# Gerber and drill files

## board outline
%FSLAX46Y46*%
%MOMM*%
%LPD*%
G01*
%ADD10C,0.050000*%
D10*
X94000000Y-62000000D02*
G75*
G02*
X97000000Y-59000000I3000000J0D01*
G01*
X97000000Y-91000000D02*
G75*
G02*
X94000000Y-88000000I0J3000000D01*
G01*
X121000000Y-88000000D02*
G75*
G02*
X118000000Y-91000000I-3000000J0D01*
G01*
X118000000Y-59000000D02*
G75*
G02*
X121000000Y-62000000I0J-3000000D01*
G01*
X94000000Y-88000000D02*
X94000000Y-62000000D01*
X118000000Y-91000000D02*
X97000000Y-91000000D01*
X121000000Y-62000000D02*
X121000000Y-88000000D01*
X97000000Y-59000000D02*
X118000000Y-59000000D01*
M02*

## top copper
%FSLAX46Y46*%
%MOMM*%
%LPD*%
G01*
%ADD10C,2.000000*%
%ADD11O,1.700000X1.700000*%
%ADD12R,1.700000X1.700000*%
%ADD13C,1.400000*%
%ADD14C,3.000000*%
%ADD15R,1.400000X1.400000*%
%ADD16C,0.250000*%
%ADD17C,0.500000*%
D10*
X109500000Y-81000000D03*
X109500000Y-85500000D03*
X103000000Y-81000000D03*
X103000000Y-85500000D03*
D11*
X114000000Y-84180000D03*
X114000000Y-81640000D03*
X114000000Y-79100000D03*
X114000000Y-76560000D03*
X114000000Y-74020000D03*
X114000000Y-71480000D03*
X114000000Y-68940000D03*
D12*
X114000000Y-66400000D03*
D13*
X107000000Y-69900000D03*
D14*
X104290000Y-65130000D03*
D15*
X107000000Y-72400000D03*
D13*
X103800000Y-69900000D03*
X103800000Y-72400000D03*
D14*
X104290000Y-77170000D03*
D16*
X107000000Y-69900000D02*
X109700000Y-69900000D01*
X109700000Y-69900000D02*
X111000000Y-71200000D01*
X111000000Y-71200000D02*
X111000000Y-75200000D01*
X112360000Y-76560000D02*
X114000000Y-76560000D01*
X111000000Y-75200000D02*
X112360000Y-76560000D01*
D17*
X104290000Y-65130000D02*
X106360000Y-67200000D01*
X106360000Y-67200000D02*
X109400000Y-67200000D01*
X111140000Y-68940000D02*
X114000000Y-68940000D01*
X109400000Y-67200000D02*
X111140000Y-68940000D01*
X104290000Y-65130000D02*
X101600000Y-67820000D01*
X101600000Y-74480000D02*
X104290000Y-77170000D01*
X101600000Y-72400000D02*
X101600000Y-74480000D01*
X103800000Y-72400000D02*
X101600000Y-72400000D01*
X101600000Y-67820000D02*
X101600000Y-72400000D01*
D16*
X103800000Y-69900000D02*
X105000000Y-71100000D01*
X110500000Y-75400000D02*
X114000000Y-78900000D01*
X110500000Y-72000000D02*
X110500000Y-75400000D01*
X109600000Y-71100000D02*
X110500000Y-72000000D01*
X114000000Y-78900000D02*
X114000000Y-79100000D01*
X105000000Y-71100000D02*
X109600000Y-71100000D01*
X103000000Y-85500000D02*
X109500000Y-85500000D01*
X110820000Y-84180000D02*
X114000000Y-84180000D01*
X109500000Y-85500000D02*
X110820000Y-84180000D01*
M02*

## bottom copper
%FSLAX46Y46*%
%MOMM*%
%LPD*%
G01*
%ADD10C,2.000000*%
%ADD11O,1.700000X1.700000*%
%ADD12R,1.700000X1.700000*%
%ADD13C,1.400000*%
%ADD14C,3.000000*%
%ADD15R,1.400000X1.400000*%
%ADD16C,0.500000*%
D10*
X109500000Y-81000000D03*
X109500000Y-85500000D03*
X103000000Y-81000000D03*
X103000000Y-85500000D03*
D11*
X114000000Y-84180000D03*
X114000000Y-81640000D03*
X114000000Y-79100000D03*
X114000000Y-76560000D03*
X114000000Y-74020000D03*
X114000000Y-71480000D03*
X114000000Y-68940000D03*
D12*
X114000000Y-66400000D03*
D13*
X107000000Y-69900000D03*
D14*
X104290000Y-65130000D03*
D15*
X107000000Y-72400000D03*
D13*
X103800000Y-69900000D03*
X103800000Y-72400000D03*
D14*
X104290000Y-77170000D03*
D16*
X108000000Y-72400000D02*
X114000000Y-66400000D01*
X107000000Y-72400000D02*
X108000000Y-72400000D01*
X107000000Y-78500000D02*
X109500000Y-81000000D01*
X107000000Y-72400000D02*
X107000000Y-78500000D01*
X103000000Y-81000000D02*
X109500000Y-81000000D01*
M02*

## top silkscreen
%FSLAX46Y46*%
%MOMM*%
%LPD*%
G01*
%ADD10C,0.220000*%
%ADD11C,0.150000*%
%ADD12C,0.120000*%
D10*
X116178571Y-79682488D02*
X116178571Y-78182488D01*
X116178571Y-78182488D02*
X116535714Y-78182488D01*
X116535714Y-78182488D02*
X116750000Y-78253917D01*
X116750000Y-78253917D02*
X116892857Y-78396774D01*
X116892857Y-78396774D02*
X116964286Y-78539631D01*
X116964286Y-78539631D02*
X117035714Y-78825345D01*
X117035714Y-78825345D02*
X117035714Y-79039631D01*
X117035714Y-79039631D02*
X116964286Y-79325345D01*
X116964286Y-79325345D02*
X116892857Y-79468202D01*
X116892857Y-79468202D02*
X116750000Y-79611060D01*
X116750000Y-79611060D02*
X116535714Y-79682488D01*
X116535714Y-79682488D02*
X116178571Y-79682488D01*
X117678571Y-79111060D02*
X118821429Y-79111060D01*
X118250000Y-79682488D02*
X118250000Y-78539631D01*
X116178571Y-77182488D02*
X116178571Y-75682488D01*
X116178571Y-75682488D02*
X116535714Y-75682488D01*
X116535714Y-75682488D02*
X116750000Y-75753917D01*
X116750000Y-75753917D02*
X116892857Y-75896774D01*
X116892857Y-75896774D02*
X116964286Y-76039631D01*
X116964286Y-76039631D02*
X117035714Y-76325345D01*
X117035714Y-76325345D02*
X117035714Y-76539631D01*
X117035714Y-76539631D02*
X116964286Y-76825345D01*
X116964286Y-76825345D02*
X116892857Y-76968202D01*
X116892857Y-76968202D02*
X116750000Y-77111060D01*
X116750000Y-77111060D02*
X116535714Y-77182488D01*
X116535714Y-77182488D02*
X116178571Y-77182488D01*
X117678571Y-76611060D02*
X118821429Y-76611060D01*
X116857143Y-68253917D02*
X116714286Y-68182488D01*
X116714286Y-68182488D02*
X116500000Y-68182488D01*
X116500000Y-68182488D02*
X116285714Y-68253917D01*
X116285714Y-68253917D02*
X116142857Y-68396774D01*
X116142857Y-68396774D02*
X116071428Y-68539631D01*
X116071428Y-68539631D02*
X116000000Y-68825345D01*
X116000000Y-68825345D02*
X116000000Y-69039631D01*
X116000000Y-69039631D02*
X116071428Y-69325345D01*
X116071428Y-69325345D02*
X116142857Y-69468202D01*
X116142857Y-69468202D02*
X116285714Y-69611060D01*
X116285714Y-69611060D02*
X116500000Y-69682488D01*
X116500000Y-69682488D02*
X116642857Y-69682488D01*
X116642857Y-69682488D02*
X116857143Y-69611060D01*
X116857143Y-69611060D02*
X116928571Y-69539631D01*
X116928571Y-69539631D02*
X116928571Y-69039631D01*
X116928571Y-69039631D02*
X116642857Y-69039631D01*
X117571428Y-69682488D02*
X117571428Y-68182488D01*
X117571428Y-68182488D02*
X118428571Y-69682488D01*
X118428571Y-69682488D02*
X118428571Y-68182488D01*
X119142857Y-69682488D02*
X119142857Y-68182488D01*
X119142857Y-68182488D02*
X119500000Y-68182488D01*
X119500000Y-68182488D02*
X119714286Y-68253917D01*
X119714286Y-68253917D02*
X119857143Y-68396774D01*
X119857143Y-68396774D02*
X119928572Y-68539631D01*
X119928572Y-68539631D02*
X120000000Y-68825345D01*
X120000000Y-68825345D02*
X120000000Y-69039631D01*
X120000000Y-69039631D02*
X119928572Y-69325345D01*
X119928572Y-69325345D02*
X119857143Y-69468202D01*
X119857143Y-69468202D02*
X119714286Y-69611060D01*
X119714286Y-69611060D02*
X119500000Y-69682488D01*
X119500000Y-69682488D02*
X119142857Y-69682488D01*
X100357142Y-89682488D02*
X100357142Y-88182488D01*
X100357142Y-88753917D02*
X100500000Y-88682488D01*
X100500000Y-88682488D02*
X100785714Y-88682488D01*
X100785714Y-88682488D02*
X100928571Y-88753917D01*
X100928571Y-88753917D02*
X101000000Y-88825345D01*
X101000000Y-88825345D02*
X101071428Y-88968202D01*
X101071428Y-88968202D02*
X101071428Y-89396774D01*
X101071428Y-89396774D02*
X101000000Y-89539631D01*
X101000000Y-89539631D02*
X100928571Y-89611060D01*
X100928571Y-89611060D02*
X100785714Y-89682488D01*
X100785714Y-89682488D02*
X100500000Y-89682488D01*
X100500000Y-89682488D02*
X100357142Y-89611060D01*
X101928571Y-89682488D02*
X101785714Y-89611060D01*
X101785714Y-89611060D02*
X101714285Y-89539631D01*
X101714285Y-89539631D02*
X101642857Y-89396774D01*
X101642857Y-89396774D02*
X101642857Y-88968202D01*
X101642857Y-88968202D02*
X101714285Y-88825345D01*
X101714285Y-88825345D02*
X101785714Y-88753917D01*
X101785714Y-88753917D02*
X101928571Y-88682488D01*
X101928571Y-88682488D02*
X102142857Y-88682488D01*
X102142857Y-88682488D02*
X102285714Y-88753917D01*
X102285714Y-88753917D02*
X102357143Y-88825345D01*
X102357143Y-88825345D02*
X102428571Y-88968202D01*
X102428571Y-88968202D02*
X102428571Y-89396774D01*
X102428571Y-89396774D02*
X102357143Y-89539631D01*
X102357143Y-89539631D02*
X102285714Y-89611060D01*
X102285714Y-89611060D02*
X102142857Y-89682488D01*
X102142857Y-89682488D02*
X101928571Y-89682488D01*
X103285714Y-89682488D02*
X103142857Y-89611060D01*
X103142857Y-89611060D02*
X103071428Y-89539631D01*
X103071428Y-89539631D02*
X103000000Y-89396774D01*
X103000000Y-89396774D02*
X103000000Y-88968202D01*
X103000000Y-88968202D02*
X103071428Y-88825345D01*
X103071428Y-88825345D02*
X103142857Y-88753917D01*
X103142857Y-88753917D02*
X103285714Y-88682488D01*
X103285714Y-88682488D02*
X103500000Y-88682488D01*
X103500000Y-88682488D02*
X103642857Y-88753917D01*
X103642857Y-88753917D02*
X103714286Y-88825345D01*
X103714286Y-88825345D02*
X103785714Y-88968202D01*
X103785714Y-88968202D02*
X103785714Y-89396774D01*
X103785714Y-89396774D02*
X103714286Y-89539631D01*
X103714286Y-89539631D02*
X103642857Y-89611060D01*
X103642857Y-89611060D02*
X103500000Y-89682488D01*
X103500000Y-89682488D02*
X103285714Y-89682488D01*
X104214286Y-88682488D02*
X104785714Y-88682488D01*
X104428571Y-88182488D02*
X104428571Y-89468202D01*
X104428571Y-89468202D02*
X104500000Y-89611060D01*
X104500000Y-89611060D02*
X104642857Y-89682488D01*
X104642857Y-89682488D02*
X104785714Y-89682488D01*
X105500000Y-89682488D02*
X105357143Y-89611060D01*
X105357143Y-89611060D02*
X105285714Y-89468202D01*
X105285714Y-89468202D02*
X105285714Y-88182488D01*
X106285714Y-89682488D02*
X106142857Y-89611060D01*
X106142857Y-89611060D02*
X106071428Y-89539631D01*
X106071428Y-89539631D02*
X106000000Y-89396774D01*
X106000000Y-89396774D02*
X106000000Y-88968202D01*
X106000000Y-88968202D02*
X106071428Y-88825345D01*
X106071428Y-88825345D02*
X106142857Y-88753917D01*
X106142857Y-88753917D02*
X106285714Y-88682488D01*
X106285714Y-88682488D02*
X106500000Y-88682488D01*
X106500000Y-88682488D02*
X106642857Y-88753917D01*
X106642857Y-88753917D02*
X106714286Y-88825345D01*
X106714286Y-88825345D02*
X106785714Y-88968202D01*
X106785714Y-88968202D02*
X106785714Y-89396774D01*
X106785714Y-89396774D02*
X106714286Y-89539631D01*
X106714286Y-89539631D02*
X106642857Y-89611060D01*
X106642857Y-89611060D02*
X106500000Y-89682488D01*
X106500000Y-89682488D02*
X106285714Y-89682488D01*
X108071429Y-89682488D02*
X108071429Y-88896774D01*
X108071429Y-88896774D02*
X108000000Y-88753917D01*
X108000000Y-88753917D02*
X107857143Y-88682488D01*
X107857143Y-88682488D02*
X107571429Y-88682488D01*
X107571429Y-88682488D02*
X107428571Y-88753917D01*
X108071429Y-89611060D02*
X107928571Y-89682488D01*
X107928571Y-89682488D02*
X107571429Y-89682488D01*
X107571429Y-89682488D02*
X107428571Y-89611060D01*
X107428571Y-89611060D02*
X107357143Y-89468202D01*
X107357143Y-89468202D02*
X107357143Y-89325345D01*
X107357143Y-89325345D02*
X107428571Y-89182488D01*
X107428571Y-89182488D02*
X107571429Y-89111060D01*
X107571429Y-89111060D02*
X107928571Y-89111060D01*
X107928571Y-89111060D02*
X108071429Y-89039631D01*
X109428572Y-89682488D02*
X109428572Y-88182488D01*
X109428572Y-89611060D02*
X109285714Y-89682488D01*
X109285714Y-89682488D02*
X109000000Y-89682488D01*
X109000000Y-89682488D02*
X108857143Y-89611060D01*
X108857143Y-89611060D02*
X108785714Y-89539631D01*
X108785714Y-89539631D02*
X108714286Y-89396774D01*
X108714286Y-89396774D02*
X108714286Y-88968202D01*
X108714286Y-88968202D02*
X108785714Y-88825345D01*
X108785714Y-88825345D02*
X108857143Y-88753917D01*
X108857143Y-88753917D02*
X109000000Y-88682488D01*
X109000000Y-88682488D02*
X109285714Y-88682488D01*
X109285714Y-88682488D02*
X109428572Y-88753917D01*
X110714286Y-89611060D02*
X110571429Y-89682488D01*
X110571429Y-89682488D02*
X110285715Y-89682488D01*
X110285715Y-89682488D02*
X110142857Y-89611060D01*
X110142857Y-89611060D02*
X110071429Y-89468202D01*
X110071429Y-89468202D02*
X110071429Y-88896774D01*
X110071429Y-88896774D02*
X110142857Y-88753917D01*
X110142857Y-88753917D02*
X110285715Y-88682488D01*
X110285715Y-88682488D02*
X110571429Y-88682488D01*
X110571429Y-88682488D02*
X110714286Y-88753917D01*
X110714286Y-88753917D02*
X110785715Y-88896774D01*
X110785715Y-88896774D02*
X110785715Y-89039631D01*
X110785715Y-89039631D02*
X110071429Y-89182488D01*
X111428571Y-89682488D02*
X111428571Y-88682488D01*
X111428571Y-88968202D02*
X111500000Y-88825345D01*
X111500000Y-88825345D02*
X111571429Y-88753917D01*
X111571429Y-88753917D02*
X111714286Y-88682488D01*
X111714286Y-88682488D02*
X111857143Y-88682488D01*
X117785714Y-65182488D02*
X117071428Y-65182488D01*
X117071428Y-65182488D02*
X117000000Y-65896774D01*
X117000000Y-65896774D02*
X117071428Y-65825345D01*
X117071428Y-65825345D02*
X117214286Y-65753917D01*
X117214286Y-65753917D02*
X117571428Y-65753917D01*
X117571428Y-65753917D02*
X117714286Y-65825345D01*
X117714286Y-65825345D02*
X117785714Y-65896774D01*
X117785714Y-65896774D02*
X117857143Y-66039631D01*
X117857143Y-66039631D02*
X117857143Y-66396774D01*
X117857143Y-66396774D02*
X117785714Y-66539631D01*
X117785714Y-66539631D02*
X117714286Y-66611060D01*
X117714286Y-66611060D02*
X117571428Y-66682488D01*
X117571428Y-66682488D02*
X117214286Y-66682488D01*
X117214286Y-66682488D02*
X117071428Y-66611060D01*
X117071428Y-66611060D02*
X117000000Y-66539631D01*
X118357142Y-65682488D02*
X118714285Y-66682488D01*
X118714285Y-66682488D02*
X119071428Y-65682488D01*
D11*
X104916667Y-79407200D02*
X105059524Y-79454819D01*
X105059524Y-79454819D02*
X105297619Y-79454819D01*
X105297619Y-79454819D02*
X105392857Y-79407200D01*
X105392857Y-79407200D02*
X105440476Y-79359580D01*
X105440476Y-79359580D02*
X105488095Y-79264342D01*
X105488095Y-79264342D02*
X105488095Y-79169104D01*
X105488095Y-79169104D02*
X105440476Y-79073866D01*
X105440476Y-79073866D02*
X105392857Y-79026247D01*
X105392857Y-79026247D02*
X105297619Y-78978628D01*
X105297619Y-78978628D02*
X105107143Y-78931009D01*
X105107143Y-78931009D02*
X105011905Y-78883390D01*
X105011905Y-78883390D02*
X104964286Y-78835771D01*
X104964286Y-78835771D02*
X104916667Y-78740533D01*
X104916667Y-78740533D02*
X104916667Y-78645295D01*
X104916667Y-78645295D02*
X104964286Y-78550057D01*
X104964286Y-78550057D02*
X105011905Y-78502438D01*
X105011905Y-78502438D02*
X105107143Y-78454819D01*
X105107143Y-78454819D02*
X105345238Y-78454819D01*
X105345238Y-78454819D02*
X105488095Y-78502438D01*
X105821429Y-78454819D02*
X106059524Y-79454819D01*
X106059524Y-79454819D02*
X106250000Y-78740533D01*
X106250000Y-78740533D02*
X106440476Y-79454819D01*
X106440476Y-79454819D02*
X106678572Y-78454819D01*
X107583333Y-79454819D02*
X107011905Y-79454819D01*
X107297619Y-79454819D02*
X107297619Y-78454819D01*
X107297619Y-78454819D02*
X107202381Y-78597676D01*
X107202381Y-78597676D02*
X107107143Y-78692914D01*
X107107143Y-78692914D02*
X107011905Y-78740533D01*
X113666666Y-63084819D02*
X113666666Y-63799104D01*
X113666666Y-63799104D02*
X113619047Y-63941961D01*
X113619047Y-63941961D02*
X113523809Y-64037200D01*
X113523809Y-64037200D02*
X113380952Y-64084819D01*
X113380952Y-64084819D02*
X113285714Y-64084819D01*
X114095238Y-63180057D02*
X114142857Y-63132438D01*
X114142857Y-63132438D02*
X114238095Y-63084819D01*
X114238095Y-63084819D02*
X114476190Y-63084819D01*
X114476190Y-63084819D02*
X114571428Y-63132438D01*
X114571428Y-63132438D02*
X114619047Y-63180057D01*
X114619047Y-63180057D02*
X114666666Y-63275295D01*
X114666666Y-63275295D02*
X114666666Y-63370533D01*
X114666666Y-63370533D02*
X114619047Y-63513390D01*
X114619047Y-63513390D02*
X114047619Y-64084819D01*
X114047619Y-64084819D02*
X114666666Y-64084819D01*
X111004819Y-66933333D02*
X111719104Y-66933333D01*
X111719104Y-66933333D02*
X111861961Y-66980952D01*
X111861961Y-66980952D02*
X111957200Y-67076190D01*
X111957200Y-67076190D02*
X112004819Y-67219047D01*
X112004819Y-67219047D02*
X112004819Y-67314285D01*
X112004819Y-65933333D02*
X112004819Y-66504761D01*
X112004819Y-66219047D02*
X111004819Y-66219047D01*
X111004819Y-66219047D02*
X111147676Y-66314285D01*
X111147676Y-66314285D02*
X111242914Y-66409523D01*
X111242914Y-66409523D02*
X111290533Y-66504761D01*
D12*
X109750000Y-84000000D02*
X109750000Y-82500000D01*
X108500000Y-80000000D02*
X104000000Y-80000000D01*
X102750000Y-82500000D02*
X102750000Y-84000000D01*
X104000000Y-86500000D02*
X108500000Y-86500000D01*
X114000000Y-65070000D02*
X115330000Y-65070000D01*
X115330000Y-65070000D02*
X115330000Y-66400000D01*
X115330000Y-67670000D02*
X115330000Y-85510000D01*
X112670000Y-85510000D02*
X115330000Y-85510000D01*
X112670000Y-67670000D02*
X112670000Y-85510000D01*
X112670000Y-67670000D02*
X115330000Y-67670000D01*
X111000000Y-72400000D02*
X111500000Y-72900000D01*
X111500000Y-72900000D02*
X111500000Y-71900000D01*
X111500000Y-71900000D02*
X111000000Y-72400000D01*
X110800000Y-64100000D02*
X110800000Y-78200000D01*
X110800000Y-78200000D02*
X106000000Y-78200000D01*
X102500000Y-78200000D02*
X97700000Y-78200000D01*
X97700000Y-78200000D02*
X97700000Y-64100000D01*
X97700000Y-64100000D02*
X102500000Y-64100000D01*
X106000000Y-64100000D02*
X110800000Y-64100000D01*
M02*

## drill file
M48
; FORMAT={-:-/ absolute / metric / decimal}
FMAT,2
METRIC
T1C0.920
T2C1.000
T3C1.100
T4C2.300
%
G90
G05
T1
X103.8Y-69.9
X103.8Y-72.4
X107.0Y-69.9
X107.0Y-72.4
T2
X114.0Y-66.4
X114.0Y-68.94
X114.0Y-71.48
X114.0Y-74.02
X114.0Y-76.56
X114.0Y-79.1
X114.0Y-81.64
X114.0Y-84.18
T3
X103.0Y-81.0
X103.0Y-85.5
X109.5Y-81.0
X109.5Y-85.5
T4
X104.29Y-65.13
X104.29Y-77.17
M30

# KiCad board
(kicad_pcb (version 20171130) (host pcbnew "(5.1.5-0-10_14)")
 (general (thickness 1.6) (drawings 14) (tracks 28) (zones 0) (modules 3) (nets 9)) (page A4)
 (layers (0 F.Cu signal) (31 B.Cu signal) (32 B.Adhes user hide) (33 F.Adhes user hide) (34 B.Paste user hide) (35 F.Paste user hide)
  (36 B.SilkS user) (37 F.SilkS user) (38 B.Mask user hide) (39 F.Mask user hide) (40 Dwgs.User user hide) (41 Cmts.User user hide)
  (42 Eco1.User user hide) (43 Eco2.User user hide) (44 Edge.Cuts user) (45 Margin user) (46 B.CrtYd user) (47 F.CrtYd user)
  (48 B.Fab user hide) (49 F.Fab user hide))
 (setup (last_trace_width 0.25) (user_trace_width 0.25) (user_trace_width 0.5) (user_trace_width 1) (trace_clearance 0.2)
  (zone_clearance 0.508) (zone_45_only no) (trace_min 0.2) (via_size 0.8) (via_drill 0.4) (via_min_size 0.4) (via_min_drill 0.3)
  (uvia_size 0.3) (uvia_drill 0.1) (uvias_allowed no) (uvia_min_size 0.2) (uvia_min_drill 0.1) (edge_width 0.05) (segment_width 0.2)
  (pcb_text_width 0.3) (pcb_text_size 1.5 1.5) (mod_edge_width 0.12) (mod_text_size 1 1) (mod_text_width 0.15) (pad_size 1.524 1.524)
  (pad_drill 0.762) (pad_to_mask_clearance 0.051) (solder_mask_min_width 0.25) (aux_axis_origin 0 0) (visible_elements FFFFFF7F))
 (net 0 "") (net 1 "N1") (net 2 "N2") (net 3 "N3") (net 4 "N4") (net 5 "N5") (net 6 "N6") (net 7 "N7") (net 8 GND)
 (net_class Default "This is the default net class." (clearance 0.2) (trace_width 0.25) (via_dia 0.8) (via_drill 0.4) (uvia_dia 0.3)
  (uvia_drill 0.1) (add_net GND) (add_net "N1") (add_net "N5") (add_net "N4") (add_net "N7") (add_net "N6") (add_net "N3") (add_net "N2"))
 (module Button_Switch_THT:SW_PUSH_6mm (layer F.Cu) (at 103 81)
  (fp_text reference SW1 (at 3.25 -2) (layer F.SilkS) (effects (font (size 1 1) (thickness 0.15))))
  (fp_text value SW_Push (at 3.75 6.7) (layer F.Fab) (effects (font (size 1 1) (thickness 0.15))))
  (fp_line (start 6.75 3) (end 6.75 1.5) (layer F.SilkS) (width 0.12))
  (fp_line (start 5.5 -1) (end 1 -1) (layer F.SilkS) (width 0.12))
  (fp_line (start -0.25 1.5) (end -0.25 3) (layer F.SilkS) (width 0.12))
  (fp_line (start 1 5.5) (end 5.5 5.5) (layer F.SilkS) (width 0.12))
  (pad 1 thru_hole circle (at 6.5 0 90) (size 2 2) (drill 1.1) (layers *.Cu *.Mask) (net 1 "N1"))
  (pad 2 thru_hole circle (at 6.5 4.5 90) (size 2 2) (drill 1.1) (layers *.Cu *.Mask) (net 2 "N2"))
  (pad 1 thru_hole circle (at 0 0 90) (size 2 2) (drill 1.1) (layers *.Cu *.Mask) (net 1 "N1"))
  (pad 2 thru_hole circle (at 0 4.5 90) (size 2 2) (drill 1.1) (layers *.Cu *.Mask) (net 2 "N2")))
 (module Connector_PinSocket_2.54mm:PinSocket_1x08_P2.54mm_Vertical (layer F.Cu) (at 114 66.4)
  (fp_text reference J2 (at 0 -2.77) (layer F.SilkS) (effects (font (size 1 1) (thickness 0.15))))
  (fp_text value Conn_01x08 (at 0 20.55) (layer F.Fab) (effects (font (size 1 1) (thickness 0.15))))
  (fp_line (start 0 -1.33) (end 1.33 -1.33) (layer F.SilkS) (width 0.12))
  (fp_line (start 1.33 -1.33) (end 1.33 0) (layer F.SilkS) (width 0.12))
  (fp_line (start 1.33 1.27) (end 1.33 19.11) (layer F.SilkS) (width 0.12))
  (fp_line (start -1.33 19.11) (end 1.33 19.11) (layer F.SilkS) (width 0.12))
  (fp_line (start -1.33 1.27) (end -1.33 19.11) (layer F.SilkS) (width 0.12))
  (fp_line (start -1.33 1.27) (end 1.33 1.27) (layer F.SilkS) (width 0.12))
  (pad 8 thru_hole oval (at 0 17.78) (size 1.7 1.7) (drill 1) (layers *.Cu *.Mask) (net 2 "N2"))
  (pad 7 thru_hole oval (at 0 15.24) (size 1.7 1.7) (drill 1) (layers *.Cu *.Mask) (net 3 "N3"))
  (pad 6 thru_hole oval (at 0 12.7) (size 1.7 1.7) (drill 1) (layers *.Cu *.Mask) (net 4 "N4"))
  (pad 5 thru_hole oval (at 0 10.16) (size 1.7 1.7) (drill 1) (layers *.Cu *.Mask) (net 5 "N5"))
  (pad 4 thru_hole oval (at 0 7.62) (size 1.7 1.7) (drill 1) (layers *.Cu *.Mask) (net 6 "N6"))
  (pad 3 thru_hole oval (at 0 5.08) (size 1.7 1.7) (drill 1) (layers *.Cu *.Mask) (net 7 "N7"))
  (pad 2 thru_hole oval (at 0 2.54) (size 1.7 1.7) (drill 1) (layers *.Cu *.Mask) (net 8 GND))
  (pad 1 thru_hole rect (at 0 0) (size 1.7 1.7) (drill 1) (layers *.Cu *.Mask) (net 1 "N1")))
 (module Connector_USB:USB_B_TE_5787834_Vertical (layer F.Cu) (at 107 72.4 270)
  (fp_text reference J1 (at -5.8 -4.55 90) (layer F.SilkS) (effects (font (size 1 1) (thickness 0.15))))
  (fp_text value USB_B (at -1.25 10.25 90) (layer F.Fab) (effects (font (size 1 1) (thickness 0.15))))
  (fp_line (start 0 -4) (end 0.5 -4.5) (layer F.SilkS) (width 0.12))
  (fp_line (start 0.5 -4.5) (end -0.5 -4.5) (layer F.SilkS) (width 0.12))
  (fp_line (start -0.5 -4.5) (end 0 -4) (layer F.SilkS) (width 0.12))
  (fp_line (start -8.3 -3.8) (end 5.8 -3.8) (layer F.SilkS) (width 0.12))
  (fp_line (start 5.8 -3.8) (end 5.8 1) (layer F.SilkS) (width 0.12))
  (fp_line (start 5.8 4.5) (end 5.8 9.3) (layer F.SilkS) (width 0.12))
  (fp_line (start 5.8 9.3) (end -8.3 9.3) (layer F.SilkS) (width 0.12))
  (fp_line (start -8.3 9.3) (end -8.3 4.5) (layer F.SilkS) (width 0.12))
  (fp_line (start -8.3 1) (end -8.3 -3.8) (layer F.SilkS) (width 0.12))
  (pad 2 thru_hole circle (at -2.5 0 270) (size 1.4 1.4) (drill 0.92) (layers *.Cu *.Mask) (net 5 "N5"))
  (pad 5 thru_hole circle (at -7.27 2.71 270) (size 3 3) (drill 2.3) (layers *.Cu *.Mask) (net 8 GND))
  (pad 1 thru_hole rect (at 0 0 270) (size 1.4 1.4) (drill 0.92) (layers *.Cu *.Mask) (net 1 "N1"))
  (pad 3 thru_hole circle (at -2.5 3.2 270) (size 1.4 1.4) (drill 0.92) (layers *.Cu *.Mask) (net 4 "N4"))
  (pad 4 thru_hole circle (at 0 3.2 270) (size 1.4 1.4) (drill 0.92) (layers *.Cu *.Mask) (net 8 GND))
  (pad 5 thru_hole circle (at 4.77 2.71 270) (size 3 3) (drill 2.3) (layers *.Cu *.Mask) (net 8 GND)))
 (gr_arc (start 97 62) (end 97 59) (angle -90) (layer Edge.Cuts) (width 0.05))
 (gr_arc (start 97 88) (end 94 88) (angle -90) (layer Edge.Cuts) (width 0.05))
 (gr_arc (start 118 88) (end 118 91) (angle -90) (layer Edge.Cuts) (width 0.05))
 (gr_arc (start 118 62) (end 121 62) (angle -90) (layer Edge.Cuts) (width 0.05))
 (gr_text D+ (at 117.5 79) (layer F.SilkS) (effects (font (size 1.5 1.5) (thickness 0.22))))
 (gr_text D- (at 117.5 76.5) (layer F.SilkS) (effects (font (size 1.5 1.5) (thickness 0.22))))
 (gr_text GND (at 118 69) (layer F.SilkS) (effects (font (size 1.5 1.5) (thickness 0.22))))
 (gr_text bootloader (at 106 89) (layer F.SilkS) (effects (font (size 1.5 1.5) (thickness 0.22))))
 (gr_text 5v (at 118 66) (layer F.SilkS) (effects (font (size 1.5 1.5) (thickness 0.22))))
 (gr_line (start 94 88) (end 94 62) (layer Edge.Cuts) (width 0.05))
 (gr_line (start 118 91) (end 97 91) (layer Edge.Cuts) (width 0.05))
 (gr_line (start 121 62) (end 121 88) (layer Edge.Cuts) (width 0.05))
 (gr_line (start 97 59) (end 118 59) (layer Edge.Cuts) (width 0.05))
 (segment (start 107 69.9) (end 109.7 69.9) (width 0.25) (layer F.Cu) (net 5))
 (segment (start 109.7 69.9) (end 111 71.2) (width 0.25) (layer F.Cu) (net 5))
 (segment (start 111 71.2) (end 111 75.2) (width 0.25) (layer F.Cu) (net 5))
 (segment (start 112.36 76.56) (end 114 76.56) (width 0.25) (layer F.Cu) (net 5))
 (segment (start 111 75.2) (end 112.36 76.56) (width 0.25) (layer F.Cu) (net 5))
 (segment (start 104.29 65.13) (end 106.36 67.2) (width 0.5) (layer F.Cu) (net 8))
 (segment (start 106.36 67.2) (end 109.4 67.2) (width 0.5) (layer F.Cu) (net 8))
 (segment (start 111.14 68.94) (end 114 68.94) (width 0.5) (layer F.Cu) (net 8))
 (segment (start 109.4 67.2) (end 111.14 68.94) (width 0.5) (layer F.Cu) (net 8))
 (segment (start 104.29 65.13) (end 101.6 67.82) (width 0.5) (layer F.Cu) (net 8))
 (segment (start 101.6 74.48) (end 104.29 77.17) (width 0.5) (layer F.Cu) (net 8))
 (segment (start 101.6 72.4) (end 101.6 74.48) (width 0.5) (layer F.Cu) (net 8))
 (segment (start 103.8 72.4) (end 101.6 72.4) (width 0.5) (layer F.Cu) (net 8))
 (segment (start 101.6 67.82) (end 101.6 72.4) (width 0.5) (layer F.Cu) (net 8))
 (segment (start 108 72.4) (end 114 66.4) (width 0.5) (layer B.Cu) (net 1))
 (segment (start 107 72.4) (end 108 72.4) (width 0.5) (layer B.Cu) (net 1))
 (segment (start 107 78.5) (end 109.5 81) (width 0.5) (layer B.Cu) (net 1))
 (segment (start 107 72.4) (end 107 78.5) (width 0.5) (layer B.Cu) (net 1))
 (segment (start 103 81) (end 109.5 81) (width 0.5) (layer B.Cu) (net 1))
 (segment (start 103.8 69.9) (end 105 71.1) (width 0.25) (layer F.Cu) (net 4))
 (segment (start 110.5 75.4) (end 114 78.9) (width 0.25) (layer F.Cu) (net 4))
 (segment (start 110.5 72) (end 110.5 75.4) (width 0.25) (layer F.Cu) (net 4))
 (segment (start 109.6 71.1) (end 110.5 72) (width 0.25) (layer F.Cu) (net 4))
 (segment (start 114 78.9) (end 114 79.1) (width 0.25) (layer F.Cu) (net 4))
 (segment (start 105 71.1) (end 109.6 71.1) (width 0.25) (layer F.Cu) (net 4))
 (segment (start 103 85.5) (end 109.5 85.5) (width 0.25) (layer F.Cu) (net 2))
 (segment (start 110.82 84.18) (end 114 84.18) (width 0.25) (layer F.Cu) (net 2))
 (segment (start 109.5 85.5) (end 110.82 84.18) (width 0.25) (layer F.Cu) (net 2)))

